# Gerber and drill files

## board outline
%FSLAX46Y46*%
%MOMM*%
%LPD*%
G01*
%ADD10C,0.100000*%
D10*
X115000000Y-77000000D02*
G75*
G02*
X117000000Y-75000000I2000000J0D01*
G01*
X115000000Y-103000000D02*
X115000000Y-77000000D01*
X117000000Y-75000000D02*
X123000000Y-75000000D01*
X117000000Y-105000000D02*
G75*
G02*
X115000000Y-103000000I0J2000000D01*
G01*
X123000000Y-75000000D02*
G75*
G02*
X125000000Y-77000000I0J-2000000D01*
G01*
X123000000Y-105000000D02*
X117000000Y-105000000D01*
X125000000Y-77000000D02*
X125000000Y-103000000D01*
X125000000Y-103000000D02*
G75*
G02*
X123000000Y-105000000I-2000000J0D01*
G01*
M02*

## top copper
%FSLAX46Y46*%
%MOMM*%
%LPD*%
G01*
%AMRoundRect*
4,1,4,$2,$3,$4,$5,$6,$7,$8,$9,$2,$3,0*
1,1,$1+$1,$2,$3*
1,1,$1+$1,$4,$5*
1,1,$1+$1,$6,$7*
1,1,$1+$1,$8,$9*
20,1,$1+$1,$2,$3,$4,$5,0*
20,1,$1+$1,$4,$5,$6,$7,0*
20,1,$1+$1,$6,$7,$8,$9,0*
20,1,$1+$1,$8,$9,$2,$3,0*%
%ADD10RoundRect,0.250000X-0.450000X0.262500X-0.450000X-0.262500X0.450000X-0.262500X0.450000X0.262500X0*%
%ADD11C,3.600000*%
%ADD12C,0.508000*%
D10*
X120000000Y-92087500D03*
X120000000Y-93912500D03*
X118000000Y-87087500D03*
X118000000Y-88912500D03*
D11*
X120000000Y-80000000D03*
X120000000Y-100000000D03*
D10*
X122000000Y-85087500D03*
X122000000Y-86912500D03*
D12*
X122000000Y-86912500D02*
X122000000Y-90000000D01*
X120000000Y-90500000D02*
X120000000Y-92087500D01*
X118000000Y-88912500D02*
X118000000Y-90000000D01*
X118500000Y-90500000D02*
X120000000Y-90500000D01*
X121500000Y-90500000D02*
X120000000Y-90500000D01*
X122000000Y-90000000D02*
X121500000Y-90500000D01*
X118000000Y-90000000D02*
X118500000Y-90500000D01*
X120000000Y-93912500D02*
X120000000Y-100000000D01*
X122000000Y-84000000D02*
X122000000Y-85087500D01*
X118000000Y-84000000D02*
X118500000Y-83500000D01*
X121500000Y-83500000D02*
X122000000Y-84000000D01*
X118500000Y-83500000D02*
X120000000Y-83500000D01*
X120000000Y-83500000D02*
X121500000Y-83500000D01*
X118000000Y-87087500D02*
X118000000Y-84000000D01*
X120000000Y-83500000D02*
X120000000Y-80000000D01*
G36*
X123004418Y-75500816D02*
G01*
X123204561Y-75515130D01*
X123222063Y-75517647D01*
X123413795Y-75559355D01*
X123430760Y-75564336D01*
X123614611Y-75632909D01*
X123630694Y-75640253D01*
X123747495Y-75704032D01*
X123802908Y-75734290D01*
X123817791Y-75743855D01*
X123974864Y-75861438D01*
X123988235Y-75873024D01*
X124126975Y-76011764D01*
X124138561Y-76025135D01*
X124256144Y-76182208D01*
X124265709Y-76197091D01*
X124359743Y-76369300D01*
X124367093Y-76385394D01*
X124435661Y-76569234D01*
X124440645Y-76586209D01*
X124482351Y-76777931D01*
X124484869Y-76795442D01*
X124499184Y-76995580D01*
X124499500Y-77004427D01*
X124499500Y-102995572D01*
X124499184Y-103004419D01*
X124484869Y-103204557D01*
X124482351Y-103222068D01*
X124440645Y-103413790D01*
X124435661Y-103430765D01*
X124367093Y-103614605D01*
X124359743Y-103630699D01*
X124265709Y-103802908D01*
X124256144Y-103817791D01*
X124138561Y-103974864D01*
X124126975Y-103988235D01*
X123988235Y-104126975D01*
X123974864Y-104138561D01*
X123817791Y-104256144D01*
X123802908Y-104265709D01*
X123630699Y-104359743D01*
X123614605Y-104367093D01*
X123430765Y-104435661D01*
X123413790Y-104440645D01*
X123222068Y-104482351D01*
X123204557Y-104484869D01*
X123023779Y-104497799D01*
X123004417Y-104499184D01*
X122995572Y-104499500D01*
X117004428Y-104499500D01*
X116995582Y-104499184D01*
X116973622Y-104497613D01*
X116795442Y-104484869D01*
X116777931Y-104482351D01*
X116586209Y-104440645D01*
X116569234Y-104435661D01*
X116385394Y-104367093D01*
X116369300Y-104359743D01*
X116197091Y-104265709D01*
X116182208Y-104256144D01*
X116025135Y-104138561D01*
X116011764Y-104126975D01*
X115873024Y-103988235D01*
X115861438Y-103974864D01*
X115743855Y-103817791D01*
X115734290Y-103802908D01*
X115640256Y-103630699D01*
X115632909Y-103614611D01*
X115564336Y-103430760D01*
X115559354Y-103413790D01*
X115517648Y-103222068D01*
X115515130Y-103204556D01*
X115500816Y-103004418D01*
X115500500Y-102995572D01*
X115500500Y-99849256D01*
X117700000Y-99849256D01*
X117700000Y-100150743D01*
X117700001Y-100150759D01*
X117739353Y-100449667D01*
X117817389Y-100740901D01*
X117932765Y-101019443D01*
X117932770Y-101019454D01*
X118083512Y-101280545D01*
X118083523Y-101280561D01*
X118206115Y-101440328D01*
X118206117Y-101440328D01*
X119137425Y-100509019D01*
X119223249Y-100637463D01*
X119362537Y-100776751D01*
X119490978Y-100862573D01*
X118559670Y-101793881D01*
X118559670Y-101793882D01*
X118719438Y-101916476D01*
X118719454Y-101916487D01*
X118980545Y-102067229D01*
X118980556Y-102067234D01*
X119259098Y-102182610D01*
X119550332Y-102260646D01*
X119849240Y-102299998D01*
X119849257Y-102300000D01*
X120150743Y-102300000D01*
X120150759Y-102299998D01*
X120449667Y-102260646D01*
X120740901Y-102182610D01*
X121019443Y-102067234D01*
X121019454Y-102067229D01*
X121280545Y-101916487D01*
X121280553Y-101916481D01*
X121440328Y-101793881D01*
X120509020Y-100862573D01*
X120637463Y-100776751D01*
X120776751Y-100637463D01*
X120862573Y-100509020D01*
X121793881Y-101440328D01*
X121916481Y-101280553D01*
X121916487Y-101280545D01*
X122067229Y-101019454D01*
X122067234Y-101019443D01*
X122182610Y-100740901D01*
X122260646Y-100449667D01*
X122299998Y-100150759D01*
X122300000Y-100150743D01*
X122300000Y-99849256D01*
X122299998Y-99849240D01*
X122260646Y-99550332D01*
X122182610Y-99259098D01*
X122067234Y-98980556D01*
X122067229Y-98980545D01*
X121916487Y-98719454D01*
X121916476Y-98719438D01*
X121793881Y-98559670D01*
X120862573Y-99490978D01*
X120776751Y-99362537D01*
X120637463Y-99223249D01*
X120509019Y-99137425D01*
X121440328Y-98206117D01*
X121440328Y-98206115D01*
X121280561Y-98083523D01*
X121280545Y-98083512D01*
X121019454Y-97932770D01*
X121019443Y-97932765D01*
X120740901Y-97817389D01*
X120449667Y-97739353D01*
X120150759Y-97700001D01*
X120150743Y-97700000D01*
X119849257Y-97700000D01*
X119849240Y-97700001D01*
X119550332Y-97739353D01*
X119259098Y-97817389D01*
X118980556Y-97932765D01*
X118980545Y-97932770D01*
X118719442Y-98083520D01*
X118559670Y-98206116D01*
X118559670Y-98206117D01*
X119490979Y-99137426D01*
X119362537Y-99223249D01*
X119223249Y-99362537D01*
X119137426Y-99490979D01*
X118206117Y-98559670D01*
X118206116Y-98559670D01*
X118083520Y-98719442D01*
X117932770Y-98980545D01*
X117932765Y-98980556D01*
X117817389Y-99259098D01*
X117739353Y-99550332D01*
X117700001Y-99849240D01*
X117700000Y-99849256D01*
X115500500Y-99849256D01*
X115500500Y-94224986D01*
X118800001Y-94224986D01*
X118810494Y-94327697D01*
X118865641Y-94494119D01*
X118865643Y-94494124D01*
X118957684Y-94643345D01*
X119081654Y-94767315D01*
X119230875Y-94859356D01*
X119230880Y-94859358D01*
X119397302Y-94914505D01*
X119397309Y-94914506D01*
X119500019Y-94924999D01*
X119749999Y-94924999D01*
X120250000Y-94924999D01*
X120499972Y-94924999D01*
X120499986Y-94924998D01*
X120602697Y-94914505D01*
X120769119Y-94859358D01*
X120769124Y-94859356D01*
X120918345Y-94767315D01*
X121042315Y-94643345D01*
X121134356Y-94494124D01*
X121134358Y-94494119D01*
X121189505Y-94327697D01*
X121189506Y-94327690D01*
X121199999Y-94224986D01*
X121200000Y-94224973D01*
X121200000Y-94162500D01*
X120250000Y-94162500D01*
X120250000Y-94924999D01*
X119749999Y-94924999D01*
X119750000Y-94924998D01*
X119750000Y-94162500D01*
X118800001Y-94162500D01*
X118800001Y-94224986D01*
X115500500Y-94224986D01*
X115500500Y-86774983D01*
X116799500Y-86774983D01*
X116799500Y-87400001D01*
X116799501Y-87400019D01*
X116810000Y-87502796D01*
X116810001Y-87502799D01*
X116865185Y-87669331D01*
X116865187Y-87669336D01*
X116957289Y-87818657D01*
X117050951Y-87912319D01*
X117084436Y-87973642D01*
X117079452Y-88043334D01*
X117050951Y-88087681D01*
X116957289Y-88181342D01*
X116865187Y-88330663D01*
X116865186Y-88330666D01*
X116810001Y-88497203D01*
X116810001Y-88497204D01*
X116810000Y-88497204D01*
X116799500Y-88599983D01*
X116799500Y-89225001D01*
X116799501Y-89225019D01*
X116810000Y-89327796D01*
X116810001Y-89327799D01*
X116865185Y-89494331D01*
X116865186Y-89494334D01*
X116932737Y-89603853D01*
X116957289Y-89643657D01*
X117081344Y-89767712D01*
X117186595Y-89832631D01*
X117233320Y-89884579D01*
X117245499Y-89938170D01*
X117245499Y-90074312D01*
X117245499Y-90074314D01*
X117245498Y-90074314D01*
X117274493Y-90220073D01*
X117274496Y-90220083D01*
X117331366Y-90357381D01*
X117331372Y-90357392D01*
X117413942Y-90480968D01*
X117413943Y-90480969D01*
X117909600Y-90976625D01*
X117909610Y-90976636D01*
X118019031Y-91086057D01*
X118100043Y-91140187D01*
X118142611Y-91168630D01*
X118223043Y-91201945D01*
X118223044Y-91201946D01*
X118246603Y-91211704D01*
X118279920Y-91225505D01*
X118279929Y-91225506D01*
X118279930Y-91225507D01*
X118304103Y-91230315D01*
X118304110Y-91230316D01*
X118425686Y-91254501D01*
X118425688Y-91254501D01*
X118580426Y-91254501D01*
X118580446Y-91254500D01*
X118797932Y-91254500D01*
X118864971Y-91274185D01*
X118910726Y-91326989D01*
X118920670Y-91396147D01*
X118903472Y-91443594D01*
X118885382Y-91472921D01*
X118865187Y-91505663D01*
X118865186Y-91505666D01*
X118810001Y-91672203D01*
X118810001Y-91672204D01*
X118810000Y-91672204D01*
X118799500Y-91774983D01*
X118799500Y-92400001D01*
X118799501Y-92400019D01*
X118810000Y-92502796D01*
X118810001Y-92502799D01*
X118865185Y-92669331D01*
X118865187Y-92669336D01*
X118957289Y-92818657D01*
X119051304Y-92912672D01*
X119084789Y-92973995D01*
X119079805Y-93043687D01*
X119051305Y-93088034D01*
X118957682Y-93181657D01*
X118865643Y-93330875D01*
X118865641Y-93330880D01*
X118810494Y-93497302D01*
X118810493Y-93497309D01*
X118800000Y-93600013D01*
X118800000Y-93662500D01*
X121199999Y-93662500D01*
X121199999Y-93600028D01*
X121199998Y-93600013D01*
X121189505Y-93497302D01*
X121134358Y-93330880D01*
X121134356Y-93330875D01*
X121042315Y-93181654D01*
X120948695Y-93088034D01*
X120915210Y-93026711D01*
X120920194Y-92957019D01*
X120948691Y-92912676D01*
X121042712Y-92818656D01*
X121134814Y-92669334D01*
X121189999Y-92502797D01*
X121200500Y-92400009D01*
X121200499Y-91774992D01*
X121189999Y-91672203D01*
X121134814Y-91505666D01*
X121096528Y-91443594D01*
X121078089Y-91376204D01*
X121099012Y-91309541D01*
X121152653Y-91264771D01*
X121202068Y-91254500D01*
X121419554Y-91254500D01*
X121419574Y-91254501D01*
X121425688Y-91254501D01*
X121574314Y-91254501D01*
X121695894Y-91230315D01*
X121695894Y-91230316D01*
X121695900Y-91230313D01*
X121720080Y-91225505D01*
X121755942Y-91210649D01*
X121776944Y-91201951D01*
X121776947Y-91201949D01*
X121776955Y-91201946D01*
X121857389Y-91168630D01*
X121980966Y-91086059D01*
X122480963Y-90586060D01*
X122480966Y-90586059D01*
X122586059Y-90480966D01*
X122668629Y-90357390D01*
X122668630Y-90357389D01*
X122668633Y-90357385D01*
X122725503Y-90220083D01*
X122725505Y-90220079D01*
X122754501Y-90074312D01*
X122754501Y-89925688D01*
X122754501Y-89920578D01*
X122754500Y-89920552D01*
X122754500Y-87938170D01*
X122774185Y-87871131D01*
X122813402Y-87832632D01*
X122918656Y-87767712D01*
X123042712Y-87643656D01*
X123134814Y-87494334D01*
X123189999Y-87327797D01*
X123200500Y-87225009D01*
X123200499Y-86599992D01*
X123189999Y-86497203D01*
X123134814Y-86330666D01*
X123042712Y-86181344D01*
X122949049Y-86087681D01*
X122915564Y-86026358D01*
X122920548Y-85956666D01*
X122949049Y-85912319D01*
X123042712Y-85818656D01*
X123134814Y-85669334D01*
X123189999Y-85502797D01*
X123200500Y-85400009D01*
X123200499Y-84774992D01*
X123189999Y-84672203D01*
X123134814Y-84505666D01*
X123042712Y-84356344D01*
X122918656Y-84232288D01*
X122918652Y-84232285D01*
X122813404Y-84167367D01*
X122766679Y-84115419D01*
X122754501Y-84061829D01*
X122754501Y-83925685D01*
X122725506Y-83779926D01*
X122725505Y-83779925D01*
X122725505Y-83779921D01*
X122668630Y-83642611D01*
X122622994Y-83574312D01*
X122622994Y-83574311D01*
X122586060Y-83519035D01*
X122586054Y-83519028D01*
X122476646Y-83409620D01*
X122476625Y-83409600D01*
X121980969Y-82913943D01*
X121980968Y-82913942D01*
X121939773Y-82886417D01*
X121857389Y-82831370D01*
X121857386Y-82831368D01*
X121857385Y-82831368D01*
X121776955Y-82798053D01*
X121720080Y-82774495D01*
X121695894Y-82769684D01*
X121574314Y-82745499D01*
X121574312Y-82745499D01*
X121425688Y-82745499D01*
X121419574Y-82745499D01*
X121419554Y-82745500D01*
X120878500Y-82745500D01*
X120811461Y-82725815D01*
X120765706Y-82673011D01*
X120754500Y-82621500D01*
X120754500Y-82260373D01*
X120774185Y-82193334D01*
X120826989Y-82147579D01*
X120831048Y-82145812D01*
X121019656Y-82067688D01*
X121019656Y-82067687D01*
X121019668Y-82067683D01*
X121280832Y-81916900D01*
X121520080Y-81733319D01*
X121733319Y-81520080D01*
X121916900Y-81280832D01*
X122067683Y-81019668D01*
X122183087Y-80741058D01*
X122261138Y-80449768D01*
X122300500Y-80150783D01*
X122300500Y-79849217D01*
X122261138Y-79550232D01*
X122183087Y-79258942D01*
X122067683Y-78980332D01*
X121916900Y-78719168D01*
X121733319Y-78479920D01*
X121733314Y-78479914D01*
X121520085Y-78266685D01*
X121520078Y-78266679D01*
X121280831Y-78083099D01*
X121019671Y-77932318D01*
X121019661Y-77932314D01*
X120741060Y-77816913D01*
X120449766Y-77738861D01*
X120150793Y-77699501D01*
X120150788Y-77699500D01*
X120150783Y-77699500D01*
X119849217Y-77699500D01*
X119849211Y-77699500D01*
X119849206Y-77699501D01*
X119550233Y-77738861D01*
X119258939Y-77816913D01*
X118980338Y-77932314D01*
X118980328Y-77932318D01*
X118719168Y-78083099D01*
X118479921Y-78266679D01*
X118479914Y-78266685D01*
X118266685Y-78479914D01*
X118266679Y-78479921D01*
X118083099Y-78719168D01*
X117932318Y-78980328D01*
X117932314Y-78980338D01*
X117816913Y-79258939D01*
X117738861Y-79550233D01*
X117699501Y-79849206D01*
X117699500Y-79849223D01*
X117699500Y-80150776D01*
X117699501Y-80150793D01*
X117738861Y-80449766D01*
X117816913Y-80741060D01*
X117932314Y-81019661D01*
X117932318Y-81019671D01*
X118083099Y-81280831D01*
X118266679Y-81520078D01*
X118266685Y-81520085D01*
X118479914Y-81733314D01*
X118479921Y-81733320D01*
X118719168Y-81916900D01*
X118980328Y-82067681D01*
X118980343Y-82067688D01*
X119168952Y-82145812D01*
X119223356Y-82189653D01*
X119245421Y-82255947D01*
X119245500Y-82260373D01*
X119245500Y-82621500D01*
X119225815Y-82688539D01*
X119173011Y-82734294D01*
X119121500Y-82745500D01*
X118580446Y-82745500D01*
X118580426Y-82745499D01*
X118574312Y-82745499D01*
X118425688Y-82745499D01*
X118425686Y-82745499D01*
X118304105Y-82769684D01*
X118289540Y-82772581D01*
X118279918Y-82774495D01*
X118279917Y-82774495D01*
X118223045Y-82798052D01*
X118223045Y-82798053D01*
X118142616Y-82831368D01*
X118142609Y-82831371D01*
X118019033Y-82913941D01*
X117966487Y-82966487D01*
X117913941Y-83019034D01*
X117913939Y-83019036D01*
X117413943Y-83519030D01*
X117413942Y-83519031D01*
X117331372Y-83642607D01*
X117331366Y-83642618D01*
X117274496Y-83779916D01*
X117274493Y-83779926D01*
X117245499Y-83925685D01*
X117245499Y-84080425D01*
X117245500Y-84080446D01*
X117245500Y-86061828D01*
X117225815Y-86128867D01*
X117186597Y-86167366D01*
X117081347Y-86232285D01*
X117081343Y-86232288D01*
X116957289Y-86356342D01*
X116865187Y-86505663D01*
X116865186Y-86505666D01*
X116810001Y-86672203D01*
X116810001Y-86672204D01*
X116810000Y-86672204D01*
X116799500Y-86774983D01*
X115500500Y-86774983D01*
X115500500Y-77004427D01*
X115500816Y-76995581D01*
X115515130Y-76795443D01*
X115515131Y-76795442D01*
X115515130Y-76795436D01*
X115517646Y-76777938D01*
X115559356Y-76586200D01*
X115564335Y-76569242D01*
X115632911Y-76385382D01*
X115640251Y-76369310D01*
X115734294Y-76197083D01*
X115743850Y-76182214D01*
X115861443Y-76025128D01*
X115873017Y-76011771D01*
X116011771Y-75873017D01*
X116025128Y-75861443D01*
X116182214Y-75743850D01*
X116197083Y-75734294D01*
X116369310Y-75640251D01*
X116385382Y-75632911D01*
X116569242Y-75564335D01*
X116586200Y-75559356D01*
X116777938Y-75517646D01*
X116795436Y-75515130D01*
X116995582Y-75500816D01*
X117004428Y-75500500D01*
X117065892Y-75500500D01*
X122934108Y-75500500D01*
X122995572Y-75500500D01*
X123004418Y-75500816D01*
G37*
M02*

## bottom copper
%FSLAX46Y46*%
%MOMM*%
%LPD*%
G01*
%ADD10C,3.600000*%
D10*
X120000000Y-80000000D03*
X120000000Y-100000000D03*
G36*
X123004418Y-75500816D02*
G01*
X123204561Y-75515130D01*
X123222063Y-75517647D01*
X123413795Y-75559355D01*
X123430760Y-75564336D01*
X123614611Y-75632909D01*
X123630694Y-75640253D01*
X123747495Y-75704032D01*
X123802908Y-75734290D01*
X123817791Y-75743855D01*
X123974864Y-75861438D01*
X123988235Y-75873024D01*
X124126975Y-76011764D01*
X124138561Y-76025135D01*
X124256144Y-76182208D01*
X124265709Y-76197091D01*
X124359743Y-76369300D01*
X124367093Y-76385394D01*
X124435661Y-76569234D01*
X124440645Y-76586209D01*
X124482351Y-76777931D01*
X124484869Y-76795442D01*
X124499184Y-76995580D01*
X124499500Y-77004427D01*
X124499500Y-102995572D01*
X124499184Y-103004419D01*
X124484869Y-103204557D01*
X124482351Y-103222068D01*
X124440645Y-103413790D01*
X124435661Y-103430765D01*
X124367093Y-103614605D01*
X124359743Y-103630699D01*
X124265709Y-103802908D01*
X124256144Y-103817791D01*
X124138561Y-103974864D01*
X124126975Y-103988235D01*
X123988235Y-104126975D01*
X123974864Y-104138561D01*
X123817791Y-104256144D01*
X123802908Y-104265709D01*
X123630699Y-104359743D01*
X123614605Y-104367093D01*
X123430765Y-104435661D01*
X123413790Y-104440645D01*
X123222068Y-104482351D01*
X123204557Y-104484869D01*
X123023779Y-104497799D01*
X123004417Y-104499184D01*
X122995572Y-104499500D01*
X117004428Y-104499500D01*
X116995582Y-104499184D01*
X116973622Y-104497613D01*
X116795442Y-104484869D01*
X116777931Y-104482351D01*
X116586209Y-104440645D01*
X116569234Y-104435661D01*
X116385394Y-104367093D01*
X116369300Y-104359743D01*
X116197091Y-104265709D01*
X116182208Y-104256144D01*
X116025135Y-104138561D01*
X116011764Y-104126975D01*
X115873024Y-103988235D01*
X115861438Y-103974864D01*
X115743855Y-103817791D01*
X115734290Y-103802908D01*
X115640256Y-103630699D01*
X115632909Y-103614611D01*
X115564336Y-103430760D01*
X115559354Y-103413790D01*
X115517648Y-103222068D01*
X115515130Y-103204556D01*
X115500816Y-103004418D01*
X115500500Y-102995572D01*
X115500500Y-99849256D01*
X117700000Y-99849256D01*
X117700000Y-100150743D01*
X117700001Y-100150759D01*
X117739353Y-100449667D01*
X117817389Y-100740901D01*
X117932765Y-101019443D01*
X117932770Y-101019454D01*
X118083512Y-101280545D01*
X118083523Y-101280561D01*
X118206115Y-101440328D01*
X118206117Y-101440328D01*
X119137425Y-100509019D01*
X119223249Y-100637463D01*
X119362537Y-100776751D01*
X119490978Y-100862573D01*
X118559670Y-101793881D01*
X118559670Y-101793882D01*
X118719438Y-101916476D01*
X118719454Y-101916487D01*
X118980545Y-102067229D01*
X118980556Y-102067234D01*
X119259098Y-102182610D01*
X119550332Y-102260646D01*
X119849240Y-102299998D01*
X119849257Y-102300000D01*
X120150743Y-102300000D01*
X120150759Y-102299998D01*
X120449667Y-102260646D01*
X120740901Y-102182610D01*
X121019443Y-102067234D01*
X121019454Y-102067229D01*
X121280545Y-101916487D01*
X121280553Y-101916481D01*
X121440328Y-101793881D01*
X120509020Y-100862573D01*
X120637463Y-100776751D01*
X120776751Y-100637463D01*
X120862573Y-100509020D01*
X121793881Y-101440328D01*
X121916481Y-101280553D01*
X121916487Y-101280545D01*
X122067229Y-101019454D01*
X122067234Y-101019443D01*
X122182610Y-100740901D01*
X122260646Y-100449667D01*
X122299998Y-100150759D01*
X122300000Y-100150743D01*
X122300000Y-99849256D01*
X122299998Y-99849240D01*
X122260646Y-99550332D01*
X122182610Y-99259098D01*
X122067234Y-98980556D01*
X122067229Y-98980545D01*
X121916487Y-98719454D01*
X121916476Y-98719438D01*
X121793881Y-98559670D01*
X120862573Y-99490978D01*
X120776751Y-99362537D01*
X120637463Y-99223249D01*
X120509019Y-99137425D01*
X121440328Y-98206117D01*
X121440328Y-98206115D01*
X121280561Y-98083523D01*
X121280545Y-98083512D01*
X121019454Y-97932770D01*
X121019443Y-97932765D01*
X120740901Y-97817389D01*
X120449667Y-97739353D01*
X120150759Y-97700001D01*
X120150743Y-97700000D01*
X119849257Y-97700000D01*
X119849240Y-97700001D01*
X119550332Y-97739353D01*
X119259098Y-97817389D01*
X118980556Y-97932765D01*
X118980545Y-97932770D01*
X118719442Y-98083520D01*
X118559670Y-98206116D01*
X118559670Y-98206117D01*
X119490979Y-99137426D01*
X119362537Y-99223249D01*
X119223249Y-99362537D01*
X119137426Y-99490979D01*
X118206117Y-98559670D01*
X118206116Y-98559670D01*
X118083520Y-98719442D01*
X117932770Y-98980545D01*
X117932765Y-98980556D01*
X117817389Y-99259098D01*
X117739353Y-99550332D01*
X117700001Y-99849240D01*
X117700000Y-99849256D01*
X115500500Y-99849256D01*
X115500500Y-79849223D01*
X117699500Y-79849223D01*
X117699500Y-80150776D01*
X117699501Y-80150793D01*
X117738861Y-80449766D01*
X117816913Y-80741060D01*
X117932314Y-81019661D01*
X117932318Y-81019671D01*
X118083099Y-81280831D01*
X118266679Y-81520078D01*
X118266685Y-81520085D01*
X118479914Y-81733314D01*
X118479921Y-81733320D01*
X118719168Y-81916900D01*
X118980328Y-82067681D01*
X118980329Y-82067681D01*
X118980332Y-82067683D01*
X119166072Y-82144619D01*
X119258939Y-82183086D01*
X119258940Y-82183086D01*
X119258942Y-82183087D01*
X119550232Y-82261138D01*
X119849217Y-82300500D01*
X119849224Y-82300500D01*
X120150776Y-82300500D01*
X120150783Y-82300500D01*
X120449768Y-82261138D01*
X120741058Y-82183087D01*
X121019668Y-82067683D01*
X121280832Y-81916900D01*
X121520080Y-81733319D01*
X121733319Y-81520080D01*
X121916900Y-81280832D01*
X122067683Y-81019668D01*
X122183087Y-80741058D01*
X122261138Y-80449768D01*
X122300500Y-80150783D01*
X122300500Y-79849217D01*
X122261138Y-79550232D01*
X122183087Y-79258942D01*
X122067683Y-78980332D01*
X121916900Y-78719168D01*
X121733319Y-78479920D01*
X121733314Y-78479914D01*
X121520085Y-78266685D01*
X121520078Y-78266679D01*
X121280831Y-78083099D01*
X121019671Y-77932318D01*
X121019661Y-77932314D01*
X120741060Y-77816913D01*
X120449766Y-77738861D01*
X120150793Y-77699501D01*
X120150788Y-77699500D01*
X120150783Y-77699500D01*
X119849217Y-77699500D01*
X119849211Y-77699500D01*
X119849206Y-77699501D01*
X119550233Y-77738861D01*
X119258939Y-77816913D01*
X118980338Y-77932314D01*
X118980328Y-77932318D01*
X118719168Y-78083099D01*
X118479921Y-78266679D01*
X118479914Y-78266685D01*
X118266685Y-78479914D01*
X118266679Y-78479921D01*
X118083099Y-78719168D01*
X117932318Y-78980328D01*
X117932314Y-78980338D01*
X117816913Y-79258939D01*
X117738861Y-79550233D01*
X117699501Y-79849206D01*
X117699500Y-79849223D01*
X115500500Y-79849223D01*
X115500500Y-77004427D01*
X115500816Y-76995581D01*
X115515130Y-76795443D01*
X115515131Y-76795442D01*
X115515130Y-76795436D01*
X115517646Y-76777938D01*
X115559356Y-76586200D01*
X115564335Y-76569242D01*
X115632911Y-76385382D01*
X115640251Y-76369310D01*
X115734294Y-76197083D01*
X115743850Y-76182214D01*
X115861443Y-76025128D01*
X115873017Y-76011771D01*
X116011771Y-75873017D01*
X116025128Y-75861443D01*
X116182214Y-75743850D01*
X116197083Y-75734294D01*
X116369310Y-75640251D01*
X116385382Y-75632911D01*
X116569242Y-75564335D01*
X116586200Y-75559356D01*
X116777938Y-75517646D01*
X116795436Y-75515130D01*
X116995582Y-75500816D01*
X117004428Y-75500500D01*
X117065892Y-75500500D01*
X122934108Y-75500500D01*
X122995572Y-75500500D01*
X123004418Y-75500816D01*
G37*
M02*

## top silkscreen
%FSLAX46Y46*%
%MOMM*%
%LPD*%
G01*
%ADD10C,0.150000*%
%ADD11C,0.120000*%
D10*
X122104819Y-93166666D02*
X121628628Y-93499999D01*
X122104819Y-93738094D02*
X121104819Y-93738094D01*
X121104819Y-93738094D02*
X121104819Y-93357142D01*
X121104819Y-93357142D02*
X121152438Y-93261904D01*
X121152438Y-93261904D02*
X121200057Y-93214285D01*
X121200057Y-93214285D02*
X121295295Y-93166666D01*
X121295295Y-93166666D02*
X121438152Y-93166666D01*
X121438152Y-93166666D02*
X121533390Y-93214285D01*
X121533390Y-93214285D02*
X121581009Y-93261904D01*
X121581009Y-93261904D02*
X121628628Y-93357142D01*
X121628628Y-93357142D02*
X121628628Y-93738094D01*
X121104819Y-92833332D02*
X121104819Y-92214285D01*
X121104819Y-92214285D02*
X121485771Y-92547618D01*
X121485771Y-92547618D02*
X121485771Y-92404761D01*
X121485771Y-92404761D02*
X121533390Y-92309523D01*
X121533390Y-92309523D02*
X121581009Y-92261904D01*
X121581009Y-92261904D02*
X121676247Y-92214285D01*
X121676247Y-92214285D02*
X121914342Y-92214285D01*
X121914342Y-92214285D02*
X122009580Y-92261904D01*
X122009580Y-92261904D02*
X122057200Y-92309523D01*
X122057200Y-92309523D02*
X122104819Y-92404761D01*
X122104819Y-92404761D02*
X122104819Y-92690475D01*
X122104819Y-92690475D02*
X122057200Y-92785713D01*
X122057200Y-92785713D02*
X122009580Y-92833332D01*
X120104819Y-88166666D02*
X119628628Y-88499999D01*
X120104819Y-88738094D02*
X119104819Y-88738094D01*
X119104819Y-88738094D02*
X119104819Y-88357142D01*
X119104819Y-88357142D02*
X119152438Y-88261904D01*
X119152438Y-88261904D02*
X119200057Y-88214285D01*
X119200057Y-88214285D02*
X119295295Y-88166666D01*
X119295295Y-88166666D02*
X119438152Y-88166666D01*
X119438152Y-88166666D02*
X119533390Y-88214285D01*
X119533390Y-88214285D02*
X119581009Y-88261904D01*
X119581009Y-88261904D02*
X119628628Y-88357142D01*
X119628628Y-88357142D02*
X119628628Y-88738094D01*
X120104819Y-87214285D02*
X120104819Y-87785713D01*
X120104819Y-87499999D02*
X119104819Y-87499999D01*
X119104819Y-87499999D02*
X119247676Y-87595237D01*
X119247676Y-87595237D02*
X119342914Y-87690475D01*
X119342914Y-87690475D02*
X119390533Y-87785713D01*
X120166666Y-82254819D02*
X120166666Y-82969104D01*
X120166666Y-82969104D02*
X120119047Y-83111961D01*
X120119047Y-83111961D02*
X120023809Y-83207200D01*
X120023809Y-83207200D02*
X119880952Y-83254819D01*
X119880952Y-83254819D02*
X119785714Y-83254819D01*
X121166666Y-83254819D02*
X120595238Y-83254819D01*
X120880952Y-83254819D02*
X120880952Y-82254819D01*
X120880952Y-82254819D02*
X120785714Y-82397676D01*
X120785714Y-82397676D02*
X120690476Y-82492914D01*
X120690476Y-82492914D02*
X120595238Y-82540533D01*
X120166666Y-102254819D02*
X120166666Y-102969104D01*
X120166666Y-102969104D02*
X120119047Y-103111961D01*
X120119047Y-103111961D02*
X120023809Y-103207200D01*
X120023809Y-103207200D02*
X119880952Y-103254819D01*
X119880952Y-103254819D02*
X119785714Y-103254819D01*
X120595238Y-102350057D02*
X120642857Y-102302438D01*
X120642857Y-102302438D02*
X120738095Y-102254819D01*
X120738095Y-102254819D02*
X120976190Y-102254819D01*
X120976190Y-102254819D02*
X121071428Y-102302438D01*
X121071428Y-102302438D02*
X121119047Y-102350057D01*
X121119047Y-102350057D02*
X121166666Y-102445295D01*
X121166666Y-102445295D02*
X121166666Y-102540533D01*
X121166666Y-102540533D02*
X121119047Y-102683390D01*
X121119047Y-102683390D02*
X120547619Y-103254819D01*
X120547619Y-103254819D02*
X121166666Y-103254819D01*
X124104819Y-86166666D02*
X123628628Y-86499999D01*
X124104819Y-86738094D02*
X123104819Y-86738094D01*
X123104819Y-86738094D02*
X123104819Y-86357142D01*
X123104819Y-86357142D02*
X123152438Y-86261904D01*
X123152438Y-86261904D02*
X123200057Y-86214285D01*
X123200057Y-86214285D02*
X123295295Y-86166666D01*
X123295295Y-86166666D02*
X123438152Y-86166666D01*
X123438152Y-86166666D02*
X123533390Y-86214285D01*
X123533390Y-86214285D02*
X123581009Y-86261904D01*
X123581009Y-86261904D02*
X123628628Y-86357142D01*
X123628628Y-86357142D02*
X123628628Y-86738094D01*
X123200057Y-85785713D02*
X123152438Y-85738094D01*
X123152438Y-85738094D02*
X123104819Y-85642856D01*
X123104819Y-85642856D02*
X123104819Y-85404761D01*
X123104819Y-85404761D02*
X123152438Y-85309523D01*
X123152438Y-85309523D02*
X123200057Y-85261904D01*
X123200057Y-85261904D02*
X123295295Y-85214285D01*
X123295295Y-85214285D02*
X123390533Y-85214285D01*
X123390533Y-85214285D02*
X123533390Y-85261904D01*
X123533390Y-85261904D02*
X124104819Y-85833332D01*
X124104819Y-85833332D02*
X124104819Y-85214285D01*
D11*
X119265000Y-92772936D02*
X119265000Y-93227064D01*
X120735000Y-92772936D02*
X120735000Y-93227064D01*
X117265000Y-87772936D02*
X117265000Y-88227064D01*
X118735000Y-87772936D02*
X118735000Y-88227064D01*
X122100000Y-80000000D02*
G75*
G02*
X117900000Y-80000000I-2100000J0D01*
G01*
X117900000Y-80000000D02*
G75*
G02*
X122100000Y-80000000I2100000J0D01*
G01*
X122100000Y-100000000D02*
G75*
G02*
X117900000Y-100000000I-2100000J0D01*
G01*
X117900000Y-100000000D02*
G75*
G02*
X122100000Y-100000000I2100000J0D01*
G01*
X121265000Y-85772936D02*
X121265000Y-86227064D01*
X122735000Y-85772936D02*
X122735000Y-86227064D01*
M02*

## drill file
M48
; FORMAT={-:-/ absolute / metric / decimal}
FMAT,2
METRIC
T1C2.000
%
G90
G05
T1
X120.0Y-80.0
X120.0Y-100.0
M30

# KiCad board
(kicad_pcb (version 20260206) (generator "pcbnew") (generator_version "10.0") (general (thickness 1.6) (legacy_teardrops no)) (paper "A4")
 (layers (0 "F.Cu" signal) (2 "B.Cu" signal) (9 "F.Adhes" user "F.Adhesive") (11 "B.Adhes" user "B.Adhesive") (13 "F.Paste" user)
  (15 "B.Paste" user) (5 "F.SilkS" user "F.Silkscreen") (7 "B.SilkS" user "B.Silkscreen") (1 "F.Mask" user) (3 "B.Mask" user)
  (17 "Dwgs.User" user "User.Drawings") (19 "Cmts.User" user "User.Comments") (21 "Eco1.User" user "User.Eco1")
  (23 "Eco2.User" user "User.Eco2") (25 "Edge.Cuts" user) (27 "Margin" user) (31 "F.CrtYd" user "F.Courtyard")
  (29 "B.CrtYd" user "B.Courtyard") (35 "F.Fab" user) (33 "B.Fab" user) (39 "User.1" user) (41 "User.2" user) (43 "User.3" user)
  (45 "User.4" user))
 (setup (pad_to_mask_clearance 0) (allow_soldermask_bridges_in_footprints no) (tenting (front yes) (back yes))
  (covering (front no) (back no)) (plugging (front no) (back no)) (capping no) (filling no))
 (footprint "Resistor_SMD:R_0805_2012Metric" (layer "F.Cu") (at 120 93 -90)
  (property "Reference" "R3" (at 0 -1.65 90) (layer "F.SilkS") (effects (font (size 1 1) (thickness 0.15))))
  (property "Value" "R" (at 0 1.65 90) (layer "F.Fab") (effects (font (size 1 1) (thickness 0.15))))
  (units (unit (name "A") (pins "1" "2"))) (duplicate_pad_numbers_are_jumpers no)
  (fp_line (start -0.227064 0.735) (end 0.227064 0.735) (stroke (width 0.12) (type solid)) (layer "F.SilkS"))
  (fp_line (start -0.227064 -0.735) (end 0.227064 -0.735) (stroke (width 0.12) (type solid)) (layer "F.SilkS"))
  (pad "1" smd roundrect (at -0.9125 0 270) (size 1.025 1.4) (layers "F.Cu" "F.Mask" "F.Paste") (roundrect_rratio 0.243902)
   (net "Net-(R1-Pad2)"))
  (pad "2" smd roundrect (at 0.9125 0 270) (size 1.025 1.4) (layers "F.Cu" "F.Mask" "F.Paste") (roundrect_rratio 0.243902) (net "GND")))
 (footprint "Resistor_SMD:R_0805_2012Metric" (layer "F.Cu") (at 118 88 -90)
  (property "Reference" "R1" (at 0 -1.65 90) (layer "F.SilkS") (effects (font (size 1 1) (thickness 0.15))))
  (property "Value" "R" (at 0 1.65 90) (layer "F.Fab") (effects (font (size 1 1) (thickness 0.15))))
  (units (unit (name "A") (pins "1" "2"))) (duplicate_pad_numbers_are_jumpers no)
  (fp_line (start -0.227064 0.735) (end 0.227064 0.735) (stroke (width 0.12) (type solid)) (layer "F.SilkS"))
  (fp_line (start -0.227064 -0.735) (end 0.227064 -0.735) (stroke (width 0.12) (type solid)) (layer "F.SilkS"))
  (pad "1" smd roundrect (at -0.9125 0 270) (size 1.025 1.4) (layers "F.Cu" "F.Mask" "F.Paste") (roundrect_rratio 0.243902)
   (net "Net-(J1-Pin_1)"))
  (pad "2" smd roundrect (at 0.9125 0 270) (size 1.025 1.4) (layers "F.Cu" "F.Mask" "F.Paste") (roundrect_rratio 0.243902)
   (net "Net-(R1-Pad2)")))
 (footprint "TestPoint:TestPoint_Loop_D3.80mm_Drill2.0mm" (layer "F.Cu") (at 120 80)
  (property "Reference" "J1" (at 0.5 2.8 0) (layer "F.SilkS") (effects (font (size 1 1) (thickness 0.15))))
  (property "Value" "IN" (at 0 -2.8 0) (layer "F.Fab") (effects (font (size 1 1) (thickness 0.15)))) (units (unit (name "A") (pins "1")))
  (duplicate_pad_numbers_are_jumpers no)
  (fp_circle (center 0 0) (end 2.1 0) (stroke (width 0.12) (type solid)) (fill no) (layer "F.SilkS"))
  (pad "1" thru_hole circle (at 0 0) (size 3.6 3.6) (drill 2) (layers "*.Cu" "*.Mask") (remove_unused_layers no) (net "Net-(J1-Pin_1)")))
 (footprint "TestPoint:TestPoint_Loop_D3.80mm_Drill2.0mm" (layer "F.Cu") (at 120 100)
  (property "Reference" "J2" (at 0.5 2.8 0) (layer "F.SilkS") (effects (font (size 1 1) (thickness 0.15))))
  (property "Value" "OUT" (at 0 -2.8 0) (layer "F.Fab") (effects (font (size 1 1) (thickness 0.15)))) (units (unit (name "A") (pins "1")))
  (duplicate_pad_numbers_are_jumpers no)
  (fp_circle (center 0 0) (end 2.1 0) (stroke (width 0.12) (type solid)) (fill no) (layer "F.SilkS"))
  (pad "1" thru_hole circle (at 0 0) (size 3.6 3.6) (drill 2) (layers "*.Cu" "*.Mask") (remove_unused_layers no) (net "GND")))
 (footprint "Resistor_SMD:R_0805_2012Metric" (layer "F.Cu") (at 122 86 -90)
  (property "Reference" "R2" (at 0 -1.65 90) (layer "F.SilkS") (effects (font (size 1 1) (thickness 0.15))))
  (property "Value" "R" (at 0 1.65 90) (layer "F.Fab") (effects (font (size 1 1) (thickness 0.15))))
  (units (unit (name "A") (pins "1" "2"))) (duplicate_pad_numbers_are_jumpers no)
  (fp_line (start -0.227064 0.735) (end 0.227064 0.735) (stroke (width 0.12) (type solid)) (layer "F.SilkS"))
  (fp_line (start -0.227064 -0.735) (end 0.227064 -0.735) (stroke (width 0.12) (type solid)) (layer "F.SilkS"))
  (pad "1" smd roundrect (at -0.9125 0 270) (size 1.025 1.4) (layers "F.Cu" "F.Mask" "F.Paste") (roundrect_rratio 0.243902)
   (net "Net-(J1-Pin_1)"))
  (pad "2" smd roundrect (at 0.9125 0 270) (size 1.025 1.4) (layers "F.Cu" "F.Mask" "F.Paste") (roundrect_rratio 0.243902)
   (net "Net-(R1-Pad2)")))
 (gr_arc (start 115 77) (mid 115.585786 75.585786) (end 117 75) (stroke (width 0.1) (type default)) (layer "Edge.Cuts"))
 (gr_line (start 115 103) (end 115 77) (stroke (width 0.1) (type default)) (layer "Edge.Cuts"))
 (gr_line (start 117 75) (end 123 75) (stroke (width 0.1) (type default)) (layer "Edge.Cuts"))
 (gr_arc (start 117 105) (mid 115.585786 104.414214) (end 115 103) (stroke (width 0.1) (type default)) (layer "Edge.Cuts"))
 (gr_arc (start 123 75) (mid 124.414214 75.585786) (end 125 77) (stroke (width 0.1) (type default)) (layer "Edge.Cuts"))
 (gr_line (start 123 105) (end 117 105) (stroke (width 0.1) (type default)) (layer "Edge.Cuts"))
 (gr_line (start 125 77) (end 125 103) (stroke (width 0.1) (type default)) (layer "Edge.Cuts"))
 (gr_arc (start 125 103) (mid 124.414214 104.414214) (end 123 105) (stroke (width 0.1) (type default)) (layer "Edge.Cuts"))
 (segment (start 122 86.9125) (end 122 90) (width 0.508) (layer "F.Cu") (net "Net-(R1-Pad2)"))
 (segment (start 120 90.5) (end 120 92.0875) (width 0.508) (layer "F.Cu") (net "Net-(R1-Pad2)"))
 (segment (start 118 88.9125) (end 118 90) (width 0.508) (layer "F.Cu") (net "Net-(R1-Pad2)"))
 (segment (start 118.5 90.5) (end 120 90.5) (width 0.508) (layer "F.Cu") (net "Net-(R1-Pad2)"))
 (segment (start 121.5 90.5) (end 120 90.5) (width 0.508) (layer "F.Cu") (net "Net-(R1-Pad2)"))
 (segment (start 122 90) (end 121.5 90.5) (width 0.508) (layer "F.Cu") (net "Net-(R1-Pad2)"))
 (segment (start 118 90) (end 118.5 90.5) (width 0.508) (layer "F.Cu") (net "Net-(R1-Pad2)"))
 (segment (start 120 93.9125) (end 120 100) (width 0.508) (layer "F.Cu") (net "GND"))
 (segment (start 122 84) (end 122 85.0875) (width 0.508) (layer "F.Cu") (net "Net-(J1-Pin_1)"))
 (segment (start 118 84) (end 118.5 83.5) (width 0.508) (layer "F.Cu") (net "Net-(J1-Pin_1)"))
 (segment (start 121.5 83.5) (end 122 84) (width 0.508) (layer "F.Cu") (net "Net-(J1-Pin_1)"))
 (segment (start 118.5 83.5) (end 120 83.5) (width 0.508) (layer "F.Cu") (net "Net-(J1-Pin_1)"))
 (segment (start 120 83.5) (end 121.5 83.5) (width 0.508) (layer "F.Cu") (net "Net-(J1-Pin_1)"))
 (segment (start 118 87.0875) (end 118 84) (width 0.508) (layer "F.Cu") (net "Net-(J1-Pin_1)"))
 (segment (start 120 83.5) (end 120 80) (width 0.508) (layer "F.Cu") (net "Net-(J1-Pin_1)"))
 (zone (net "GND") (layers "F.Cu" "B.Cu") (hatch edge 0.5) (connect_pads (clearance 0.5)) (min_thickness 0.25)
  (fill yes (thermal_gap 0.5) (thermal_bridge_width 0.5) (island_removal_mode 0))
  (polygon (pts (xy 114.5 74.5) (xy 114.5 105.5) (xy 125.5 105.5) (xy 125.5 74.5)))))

